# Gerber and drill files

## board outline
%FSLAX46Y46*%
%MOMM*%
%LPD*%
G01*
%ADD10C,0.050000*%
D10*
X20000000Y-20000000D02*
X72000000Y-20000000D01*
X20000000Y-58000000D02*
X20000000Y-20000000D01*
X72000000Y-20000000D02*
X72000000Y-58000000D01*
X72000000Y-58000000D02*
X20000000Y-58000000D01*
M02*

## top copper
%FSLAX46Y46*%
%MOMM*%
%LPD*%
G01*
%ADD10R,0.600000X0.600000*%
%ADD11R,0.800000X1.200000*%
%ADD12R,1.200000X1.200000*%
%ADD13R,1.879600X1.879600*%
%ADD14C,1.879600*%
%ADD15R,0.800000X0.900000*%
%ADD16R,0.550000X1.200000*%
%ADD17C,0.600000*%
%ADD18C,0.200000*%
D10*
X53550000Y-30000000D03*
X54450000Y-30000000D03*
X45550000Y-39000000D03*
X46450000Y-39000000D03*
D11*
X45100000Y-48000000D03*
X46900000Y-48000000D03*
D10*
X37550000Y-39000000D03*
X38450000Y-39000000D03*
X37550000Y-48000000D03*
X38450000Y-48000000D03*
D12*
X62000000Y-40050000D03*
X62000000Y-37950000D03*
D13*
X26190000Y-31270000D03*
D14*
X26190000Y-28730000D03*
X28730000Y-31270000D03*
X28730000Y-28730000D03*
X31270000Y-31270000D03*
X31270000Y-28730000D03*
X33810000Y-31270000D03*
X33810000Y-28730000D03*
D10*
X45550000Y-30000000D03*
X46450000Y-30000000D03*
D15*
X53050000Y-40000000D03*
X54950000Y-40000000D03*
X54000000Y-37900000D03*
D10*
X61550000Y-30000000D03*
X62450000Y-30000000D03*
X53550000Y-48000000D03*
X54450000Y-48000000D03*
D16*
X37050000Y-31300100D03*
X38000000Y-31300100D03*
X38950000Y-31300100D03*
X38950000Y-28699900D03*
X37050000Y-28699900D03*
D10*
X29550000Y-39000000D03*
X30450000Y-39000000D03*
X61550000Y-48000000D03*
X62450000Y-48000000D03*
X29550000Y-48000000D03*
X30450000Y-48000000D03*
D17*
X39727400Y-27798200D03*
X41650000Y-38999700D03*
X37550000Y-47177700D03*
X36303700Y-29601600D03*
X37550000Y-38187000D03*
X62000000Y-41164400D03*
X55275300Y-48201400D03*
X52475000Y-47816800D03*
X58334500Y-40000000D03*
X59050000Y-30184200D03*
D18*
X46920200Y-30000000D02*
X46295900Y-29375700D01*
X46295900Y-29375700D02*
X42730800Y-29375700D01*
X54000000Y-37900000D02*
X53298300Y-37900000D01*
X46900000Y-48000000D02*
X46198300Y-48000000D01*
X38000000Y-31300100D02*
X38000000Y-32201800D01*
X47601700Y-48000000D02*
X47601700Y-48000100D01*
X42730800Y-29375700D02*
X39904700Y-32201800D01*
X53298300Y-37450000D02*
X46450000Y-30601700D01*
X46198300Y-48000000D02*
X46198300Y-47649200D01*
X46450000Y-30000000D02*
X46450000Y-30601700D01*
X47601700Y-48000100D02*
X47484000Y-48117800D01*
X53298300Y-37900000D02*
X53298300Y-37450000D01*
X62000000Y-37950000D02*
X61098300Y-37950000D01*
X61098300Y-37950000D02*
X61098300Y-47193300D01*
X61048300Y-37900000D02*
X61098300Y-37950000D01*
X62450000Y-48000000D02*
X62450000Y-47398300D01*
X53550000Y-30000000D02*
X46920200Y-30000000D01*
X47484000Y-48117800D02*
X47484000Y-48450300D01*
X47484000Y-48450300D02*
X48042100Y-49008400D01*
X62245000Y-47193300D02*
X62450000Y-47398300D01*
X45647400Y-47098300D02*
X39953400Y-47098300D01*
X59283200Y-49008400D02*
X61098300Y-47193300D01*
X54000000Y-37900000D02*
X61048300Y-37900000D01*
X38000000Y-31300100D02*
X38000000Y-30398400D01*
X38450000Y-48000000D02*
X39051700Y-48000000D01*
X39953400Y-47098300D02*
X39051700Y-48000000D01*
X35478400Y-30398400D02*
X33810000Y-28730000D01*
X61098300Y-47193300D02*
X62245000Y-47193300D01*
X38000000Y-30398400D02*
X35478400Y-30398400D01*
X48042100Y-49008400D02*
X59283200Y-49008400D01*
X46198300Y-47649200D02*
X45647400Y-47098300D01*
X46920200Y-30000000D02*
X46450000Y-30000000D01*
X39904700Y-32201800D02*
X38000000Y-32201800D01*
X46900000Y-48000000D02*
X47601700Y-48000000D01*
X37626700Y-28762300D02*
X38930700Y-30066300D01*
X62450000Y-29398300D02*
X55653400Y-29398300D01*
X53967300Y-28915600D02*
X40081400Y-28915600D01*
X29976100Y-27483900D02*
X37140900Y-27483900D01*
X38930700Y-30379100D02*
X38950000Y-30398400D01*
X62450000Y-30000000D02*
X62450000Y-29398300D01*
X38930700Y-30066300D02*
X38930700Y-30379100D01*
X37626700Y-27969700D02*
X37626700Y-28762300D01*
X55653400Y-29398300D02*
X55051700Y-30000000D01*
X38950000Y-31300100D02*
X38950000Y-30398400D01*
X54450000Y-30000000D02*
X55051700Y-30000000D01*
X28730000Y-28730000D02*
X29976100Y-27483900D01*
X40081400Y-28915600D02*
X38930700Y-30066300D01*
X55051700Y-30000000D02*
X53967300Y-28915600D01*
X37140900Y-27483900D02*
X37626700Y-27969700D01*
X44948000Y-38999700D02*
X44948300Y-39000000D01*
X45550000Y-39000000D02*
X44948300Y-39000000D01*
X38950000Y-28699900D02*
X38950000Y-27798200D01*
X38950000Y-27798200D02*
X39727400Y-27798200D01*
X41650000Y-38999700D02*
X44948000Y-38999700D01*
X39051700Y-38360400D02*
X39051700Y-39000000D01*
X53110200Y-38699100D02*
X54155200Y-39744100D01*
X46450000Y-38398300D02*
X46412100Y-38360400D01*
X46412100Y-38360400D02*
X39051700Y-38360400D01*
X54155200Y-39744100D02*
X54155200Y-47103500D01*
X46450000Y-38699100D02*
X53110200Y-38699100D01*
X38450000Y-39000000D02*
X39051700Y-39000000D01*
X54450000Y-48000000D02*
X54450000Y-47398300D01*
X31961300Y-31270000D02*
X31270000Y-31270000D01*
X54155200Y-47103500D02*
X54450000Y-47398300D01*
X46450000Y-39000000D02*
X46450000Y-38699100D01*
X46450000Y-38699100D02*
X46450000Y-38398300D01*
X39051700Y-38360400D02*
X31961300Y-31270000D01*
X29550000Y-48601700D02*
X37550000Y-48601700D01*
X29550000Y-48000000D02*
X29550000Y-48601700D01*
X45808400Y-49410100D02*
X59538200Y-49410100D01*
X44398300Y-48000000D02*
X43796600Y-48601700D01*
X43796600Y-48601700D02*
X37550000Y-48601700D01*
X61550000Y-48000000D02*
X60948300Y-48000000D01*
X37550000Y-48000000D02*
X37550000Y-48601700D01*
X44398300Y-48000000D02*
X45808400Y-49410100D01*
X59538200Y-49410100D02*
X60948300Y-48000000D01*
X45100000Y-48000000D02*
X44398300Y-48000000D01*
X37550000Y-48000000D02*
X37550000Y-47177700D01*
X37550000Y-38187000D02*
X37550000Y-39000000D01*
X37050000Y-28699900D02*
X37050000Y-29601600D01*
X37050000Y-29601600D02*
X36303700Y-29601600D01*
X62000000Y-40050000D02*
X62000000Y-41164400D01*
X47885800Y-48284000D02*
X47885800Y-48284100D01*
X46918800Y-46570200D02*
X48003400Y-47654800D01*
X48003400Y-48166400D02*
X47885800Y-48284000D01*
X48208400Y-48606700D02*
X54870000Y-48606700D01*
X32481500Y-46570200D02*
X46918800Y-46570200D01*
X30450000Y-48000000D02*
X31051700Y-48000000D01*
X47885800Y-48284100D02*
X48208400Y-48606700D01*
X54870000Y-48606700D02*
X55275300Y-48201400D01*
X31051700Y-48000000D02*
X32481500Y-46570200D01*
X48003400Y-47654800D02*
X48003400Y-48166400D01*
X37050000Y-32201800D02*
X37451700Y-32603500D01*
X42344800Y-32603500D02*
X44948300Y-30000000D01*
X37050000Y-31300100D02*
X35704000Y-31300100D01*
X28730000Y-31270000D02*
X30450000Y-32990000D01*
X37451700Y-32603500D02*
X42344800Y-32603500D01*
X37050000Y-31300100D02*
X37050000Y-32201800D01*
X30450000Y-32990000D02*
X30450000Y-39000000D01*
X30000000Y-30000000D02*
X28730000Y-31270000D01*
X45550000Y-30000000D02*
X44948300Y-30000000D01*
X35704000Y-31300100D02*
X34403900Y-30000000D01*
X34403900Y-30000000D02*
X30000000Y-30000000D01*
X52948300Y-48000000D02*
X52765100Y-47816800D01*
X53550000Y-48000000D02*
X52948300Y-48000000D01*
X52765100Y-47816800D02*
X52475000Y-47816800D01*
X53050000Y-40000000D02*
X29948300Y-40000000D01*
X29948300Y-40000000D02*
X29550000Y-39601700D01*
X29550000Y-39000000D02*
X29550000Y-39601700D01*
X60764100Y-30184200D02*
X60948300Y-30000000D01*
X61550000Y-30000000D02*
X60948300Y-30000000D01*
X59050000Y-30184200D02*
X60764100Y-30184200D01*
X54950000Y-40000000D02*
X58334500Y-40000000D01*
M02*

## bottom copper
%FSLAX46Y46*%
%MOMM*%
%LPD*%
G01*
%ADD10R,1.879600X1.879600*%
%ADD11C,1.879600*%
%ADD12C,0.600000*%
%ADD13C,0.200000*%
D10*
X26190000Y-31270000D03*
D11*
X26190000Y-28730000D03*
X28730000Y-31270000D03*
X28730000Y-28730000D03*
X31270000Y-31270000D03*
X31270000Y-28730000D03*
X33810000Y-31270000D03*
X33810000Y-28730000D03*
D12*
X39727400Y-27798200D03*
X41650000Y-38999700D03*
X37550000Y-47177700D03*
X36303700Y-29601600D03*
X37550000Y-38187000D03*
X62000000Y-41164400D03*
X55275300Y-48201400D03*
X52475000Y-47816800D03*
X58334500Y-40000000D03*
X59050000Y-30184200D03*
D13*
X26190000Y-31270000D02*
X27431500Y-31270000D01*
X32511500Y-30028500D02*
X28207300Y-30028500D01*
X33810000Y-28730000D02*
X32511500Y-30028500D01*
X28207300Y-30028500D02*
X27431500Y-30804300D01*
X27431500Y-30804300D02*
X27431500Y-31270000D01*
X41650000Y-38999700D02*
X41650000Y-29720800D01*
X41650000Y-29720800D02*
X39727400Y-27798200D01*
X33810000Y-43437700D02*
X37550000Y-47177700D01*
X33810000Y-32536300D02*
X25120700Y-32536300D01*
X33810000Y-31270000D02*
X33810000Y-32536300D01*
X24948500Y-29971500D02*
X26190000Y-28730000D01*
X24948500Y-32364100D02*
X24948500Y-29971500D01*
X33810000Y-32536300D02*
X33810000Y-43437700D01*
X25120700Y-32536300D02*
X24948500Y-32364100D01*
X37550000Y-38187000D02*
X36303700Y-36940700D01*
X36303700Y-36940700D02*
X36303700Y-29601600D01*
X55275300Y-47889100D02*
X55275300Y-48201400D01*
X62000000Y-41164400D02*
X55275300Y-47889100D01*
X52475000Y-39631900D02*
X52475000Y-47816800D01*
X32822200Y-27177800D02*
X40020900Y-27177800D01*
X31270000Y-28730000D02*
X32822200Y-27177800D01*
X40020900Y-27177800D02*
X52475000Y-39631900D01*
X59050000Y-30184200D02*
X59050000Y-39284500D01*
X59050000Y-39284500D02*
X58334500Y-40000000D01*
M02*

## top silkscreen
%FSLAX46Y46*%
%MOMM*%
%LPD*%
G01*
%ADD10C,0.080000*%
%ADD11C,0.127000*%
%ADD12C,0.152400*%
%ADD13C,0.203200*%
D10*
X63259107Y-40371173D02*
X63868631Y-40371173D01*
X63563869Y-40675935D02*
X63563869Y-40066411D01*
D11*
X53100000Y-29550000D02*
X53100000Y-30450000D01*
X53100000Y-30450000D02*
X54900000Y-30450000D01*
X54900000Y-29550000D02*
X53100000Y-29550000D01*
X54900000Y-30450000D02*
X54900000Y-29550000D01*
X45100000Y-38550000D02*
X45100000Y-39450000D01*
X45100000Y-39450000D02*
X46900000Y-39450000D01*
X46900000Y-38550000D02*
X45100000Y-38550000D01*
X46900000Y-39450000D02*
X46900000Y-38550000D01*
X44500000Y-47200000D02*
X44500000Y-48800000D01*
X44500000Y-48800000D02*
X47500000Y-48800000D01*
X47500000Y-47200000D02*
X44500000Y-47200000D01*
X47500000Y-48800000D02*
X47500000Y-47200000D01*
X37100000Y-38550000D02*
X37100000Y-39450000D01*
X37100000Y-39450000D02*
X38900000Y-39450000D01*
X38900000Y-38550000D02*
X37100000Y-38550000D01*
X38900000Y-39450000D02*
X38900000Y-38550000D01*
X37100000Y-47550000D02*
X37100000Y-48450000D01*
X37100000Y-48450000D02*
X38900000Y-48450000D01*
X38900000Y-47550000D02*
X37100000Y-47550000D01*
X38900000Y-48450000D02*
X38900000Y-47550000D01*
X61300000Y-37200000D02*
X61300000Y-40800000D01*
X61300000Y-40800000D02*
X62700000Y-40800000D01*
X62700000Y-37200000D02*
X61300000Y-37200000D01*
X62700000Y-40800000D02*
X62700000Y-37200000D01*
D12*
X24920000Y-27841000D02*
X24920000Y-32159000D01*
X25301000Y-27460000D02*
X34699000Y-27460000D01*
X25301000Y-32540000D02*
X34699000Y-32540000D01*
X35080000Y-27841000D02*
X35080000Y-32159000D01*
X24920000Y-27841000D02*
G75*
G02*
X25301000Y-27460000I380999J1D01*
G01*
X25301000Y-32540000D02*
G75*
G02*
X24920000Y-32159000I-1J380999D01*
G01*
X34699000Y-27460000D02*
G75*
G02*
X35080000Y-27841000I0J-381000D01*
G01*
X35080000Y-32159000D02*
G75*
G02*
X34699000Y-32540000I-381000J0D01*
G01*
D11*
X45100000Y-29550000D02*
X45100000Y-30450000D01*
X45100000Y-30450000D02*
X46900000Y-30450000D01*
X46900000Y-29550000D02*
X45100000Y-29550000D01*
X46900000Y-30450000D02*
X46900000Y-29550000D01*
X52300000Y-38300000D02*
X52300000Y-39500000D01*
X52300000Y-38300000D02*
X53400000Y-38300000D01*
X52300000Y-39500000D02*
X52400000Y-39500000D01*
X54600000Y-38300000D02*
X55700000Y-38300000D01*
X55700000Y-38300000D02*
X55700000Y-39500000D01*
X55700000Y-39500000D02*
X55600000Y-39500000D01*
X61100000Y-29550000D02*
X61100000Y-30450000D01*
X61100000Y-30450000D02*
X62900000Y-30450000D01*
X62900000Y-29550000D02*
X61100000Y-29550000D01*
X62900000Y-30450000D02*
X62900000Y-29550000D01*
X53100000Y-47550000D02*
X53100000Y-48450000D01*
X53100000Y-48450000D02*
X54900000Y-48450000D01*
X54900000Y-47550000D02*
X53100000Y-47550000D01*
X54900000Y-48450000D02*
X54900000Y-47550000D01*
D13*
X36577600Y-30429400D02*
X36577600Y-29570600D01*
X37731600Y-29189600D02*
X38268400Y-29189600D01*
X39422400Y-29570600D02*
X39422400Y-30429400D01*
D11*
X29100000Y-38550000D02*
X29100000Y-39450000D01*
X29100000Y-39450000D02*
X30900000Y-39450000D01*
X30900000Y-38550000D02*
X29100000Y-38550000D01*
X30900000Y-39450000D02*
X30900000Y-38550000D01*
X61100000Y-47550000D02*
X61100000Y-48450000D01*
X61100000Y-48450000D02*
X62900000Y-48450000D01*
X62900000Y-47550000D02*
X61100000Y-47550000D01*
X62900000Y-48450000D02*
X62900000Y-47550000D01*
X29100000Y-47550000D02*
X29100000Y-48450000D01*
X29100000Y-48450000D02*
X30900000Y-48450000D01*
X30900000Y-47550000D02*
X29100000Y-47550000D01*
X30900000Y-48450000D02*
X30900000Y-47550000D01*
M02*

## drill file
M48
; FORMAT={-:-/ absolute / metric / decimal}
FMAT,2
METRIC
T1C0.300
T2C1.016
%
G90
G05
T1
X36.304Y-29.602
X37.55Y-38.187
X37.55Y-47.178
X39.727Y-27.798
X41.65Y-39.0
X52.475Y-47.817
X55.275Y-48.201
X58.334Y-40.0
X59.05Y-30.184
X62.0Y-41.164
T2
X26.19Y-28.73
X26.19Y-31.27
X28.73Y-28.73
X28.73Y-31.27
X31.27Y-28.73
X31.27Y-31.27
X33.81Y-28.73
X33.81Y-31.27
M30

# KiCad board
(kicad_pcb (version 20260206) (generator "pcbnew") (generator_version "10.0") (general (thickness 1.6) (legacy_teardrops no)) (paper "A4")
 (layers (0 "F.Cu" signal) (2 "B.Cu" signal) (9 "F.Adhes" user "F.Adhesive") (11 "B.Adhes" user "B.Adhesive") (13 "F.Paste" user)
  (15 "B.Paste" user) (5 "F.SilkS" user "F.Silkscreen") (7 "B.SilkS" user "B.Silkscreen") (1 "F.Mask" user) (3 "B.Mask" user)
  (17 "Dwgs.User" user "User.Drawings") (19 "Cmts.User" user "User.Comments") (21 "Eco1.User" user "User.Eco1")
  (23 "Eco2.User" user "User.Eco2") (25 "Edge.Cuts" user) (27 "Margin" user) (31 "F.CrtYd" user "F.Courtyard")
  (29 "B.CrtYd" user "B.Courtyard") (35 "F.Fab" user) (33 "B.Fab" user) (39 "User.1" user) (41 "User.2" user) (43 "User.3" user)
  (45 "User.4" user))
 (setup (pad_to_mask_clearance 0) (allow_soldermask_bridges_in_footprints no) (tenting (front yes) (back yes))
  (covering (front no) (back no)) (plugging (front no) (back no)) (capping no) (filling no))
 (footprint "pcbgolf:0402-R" (layer "F.Cu") (at 54 30)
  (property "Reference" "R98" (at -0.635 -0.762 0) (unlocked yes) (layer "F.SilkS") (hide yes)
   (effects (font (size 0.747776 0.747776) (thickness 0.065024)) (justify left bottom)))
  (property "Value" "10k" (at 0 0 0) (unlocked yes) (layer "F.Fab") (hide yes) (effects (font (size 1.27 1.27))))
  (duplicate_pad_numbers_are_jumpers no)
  (fp_line (start -0.9 -0.45) (end -0.9 0.45) (stroke (width 0.127) (type solid)) (layer "F.SilkS"))
  (fp_line (start -0.9 0.45) (end 0.9 0.45) (stroke (width 0.127) (type solid)) (layer "F.SilkS"))
  (fp_line (start 0.9 -0.45) (end -0.9 -0.45) (stroke (width 0.127) (type solid)) (layer "F.SilkS"))
  (fp_line (start 0.9 0.45) (end 0.9 -0.45) (stroke (width 0.127) (type solid)) (layer "F.SilkS"))
  (pad "1" smd rect (at -0.45 0) (size 0.6 0.6) (layers "F.Cu" "F.Mask" "F.Paste") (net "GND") (solder_mask_margin 0.0508)
   (solder_paste_margin 0) (thermal_bridge_angle 0))
  (pad "2" smd rect (at 0.45 0) (size 0.6 0.6) (layers "F.Cu" "F.Mask" "F.Paste") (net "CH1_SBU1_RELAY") (solder_mask_margin 0.0508)
   (solder_paste_margin 0) (thermal_bridge_angle 0)))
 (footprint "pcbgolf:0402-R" (layer "F.Cu") (at 46 39)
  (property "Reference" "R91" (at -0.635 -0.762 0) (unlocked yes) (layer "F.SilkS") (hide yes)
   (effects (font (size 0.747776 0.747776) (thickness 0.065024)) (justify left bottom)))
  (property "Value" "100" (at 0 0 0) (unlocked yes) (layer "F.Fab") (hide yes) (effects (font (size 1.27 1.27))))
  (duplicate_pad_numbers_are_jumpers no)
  (fp_line (start -0.9 -0.45) (end -0.9 0.45) (stroke (width 0.127) (type solid)) (layer "F.SilkS"))
  (fp_line (start -0.9 0.45) (end 0.9 0.45) (stroke (width 0.127) (type solid)) (layer "F.SilkS"))
  (fp_line (start 0.9 -0.45) (end -0.9 -0.45) (stroke (width 0.127) (type solid)) (layer "F.SilkS"))
  (fp_line (start 0.9 0.45) (end 0.9 -0.45) (stroke (width 0.127) (type solid)) (layer "F.SilkS"))
  (pad "1" smd rect (at -0.45 0) (size 0.6 0.6) (layers "F.Cu" "F.Mask" "F.Paste") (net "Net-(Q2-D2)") (solder_mask_margin 0.0508)
   (solder_paste_margin 0) (thermal_bridge_angle 0))
  (pad "2" smd rect (at 0.45 0) (size 0.6 0.6) (layers "F.Cu" "F.Mask" "F.Paste") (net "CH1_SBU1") (solder_mask_margin 0.0508)
   (solder_paste_margin 0) (thermal_bridge_angle 0)))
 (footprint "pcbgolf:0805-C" (layer "F.Cu") (at 46 48)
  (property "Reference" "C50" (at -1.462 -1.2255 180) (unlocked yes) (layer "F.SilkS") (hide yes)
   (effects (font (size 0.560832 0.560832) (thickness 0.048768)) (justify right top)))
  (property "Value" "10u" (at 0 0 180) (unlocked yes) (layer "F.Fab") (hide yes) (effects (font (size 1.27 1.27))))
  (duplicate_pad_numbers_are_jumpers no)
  (fp_line (start -1.5 -0.8) (end -1.5 0.8) (stroke (width 0.127) (type solid)) (layer "F.SilkS"))
  (fp_line (start -1.5 0.8) (end 1.5 0.8) (stroke (width 0.127) (type solid)) (layer "F.SilkS"))
  (fp_line (start 1.5 -0.8) (end -1.5 -0.8) (stroke (width 0.127) (type solid)) (layer "F.SilkS"))
  (fp_line (start 1.5 0.8) (end 1.5 -0.8) (stroke (width 0.127) (type solid)) (layer "F.SilkS"))
  (pad "1" smd rect (at -0.9 0) (size 0.8 1.2) (layers "F.Cu" "F.Mask" "F.Paste") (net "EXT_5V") (solder_mask_margin 0.0508)
   (solder_paste_margin 0) (thermal_bridge_angle 0))
  (pad "2" smd rect (at 0.9 0) (size 0.8 1.2) (layers "F.Cu" "F.Mask" "F.Paste") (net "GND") (solder_mask_margin 0.0508)
   (solder_paste_margin 0) (thermal_bridge_angle 0)))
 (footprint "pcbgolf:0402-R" (layer "F.Cu") (at 38 39)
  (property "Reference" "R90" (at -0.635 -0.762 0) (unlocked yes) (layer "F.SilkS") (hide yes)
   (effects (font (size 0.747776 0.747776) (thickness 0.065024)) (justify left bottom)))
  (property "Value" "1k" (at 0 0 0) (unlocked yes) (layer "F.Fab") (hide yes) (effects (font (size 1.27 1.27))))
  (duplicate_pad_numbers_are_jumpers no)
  (fp_line (start -0.9 -0.45) (end -0.9 0.45) (stroke (width 0.127) (type solid)) (layer "F.SilkS"))
  (fp_line (start -0.9 0.45) (end 0.9 0.45) (stroke (width 0.127) (type solid)) (layer "F.SilkS"))
  (fp_line (start 0.9 -0.45) (end -0.9 -0.45) (stroke (width 0.127) (type solid)) (layer "F.SilkS"))
  (fp_line (start 0.9 0.45) (end 0.9 -0.45) (stroke (width 0.127) (type solid)) (layer "F.SilkS"))
  (pad "1" smd rect (at -0.45 0) (size 0.6 0.6) (layers "F.Cu" "F.Mask" "F.Paste") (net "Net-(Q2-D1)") (solder_mask_margin 0.0508)
   (solder_paste_margin 0) (thermal_bridge_angle 0))
  (pad "2" smd rect (at 0.45 0) (size 0.6 0.6) (layers "F.Cu" "F.Mask" "F.Paste") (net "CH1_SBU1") (solder_mask_margin 0.0508)
   (solder_paste_margin 0) (thermal_bridge_angle 0)))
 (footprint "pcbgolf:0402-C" (layer "F.Cu") (at 38 48)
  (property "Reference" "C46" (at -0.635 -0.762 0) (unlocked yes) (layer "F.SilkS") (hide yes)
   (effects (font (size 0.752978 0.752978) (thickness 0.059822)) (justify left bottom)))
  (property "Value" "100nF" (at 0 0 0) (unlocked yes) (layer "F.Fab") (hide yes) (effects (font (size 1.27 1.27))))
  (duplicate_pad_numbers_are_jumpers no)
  (fp_line (start -0.9 -0.45) (end -0.9 0.45) (stroke (width 0.127) (type solid)) (layer "F.SilkS"))
  (fp_line (start -0.9 0.45) (end 0.9 0.45) (stroke (width 0.127) (type solid)) (layer "F.SilkS"))
  (fp_line (start 0.9 -0.45) (end -0.9 -0.45) (stroke (width 0.127) (type solid)) (layer "F.SilkS"))
  (fp_line (start 0.9 0.45) (end 0.9 -0.45) (stroke (width 0.127) (type solid)) (layer "F.SilkS"))
  (pad "1" smd rect (at -0.45 0) (size 0.6 0.6) (layers "F.Cu" "F.Mask" "F.Paste") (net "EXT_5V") (solder_mask_margin 0.0508)
   (solder_paste_margin 0) (thermal_bridge_angle 0))
  (pad "2" smd rect (at 0.45 0) (size 0.6 0.6) (layers "F.Cu" "F.Mask" "F.Paste") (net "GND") (solder_mask_margin 0.0508)
   (solder_paste_margin 0) (thermal_bridge_angle 0)))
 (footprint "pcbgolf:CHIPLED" (layer "F.Cu") (at 62 39)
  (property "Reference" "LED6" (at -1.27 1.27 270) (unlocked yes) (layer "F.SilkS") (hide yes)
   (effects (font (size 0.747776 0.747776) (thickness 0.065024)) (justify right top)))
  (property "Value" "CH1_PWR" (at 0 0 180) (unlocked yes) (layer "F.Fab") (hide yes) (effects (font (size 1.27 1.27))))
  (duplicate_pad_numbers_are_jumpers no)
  (fp_line (start -0.7 -1.8) (end -0.7 1.8) (stroke (width 0.127) (type solid)) (layer "F.SilkS"))
  (fp_line (start -0.7 1.8) (end 0.7 1.8) (stroke (width 0.127) (type solid)) (layer "F.SilkS"))
  (fp_line (start 0.7 -1.8) (end -0.7 -1.8) (stroke (width 0.127) (type solid)) (layer "F.SilkS"))
  (fp_line (start 0.7 1.8) (end 0.7 -1.8) (stroke (width 0.127) (type solid)) (layer "F.SilkS"))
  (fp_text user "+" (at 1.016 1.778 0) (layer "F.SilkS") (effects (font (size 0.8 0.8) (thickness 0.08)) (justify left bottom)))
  (pad "A" smd rect (at 0 1.05) (size 1.2 1.2) (layers "F.Cu" "F.Mask" "F.Paste") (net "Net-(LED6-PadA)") (solder_mask_margin 0.0508)
   (solder_paste_margin 0) (thermal_bridge_angle 0))
  (pad "C" smd rect (at 0 -1.05) (size 1.2 1.2) (layers "F.Cu" "F.Mask" "F.Paste") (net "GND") (solder_mask_margin 0.0508)
   (solder_paste_margin 0) (thermal_bridge_angle 0)))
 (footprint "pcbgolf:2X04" (layer "F.Cu") (at 30 30)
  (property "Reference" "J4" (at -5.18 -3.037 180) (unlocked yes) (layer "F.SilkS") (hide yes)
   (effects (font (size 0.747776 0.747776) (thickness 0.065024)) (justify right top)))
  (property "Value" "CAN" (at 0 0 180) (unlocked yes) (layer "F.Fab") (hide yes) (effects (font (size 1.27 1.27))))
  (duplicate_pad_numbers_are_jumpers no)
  (fp_line (start -5.08 -2.159) (end -5.08 2.159) (stroke (width 0.1524) (type solid)) (layer "F.SilkS"))
  (fp_line (start -4.699 -2.54) (end 4.699 -2.54) (stroke (width 0.1524) (type solid)) (layer "F.SilkS"))
  (fp_line (start -4.699 2.54) (end 4.699 2.54) (stroke (width 0.1524) (type solid)) (layer "F.SilkS"))
  (fp_line (start 5.08 -2.159) (end 5.08 2.159) (stroke (width 0.1524) (type solid)) (layer "F.SilkS"))
  (fp_arc (start -5.08 -2.159) (mid -4.968408 -2.428408) (end -4.699 -2.54) (stroke (width 0.1524) (type solid)) (layer "F.SilkS"))
  (fp_arc (start -4.699 2.54) (mid -4.968408 2.428408) (end -5.08 2.159) (stroke (width 0.1524) (type solid)) (layer "F.SilkS"))
  (fp_arc (start 4.699 -2.54) (mid 4.968408 -2.428408) (end 5.08 -2.159) (stroke (width 0.1524) (type solid)) (layer "F.SilkS"))
  (fp_arc (start 5.08 2.159) (mid 4.968408 2.428408) (end 4.699 2.54) (stroke (width 0.1524) (type solid)) (layer "F.SilkS"))
  (pad "1" thru_hole rect (at -3.81 1.27 90) (size 1.8796 1.8796) (drill 1.016) (layers "*.Cu" "*.Mask") (remove_unused_layers no)
   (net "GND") (solder_mask_margin 0.0508) (thermal_bridge_angle 0))
  (pad "2" thru_hole circle (at -3.81 -1.27 90) (size 1.8796 1.8796) (drill 1.016) (layers "*.Cu" "*.Mask") (remove_unused_layers no)
   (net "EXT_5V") (solder_mask_margin 0.0508) (thermal_bridge_angle 0))
  (pad "3" thru_hole circle (at -1.27 1.27 90) (size 1.8796 1.8796) (drill 1.016) (layers "*.Cu" "*.Mask") (remove_unused_layers no)
   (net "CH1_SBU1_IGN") (solder_mask_margin 0.0508) (thermal_bridge_angle 0))
  (pad "4" thru_hole circle (at -1.27 -1.27 90) (size 1.8796 1.8796) (drill 1.016) (layers "*.Cu" "*.Mask") (remove_unused_layers no)
   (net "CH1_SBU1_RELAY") (solder_mask_margin 0.0508) (thermal_bridge_angle 0))
  (pad "5" thru_hole circle (at 1.27 1.27 90) (size 1.8796 1.8796) (drill 1.016) (layers "*.Cu" "*.Mask") (remove_unused_layers no)
   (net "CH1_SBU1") (solder_mask_margin 0.0508) (thermal_bridge_angle 0))
  (pad "6" thru_hole circle (at 1.27 -1.27 90) (size 1.8796 1.8796) (drill 1.016) (layers "*.Cu" "*.Mask") (remove_unused_layers no)
   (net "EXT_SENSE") (solder_mask_margin 0.0508) (thermal_bridge_angle 0))
  (pad "7" thru_hole circle (at 3.81 1.27 90) (size 1.8796 1.8796) (drill 1.016) (layers "*.Cu" "*.Mask") (remove_unused_layers no)
   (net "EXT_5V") (solder_mask_margin 0.0508) (thermal_bridge_angle 0))
  (pad "8" thru_hole circle (at 3.81 -1.27 90) (size 1.8796 1.8796) (drill 1.016) (layers "*.Cu" "*.Mask") (remove_unused_layers no)
   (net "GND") (solder_mask_margin 0.0508) (thermal_bridge_angle 0)))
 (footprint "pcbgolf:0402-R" (layer "F.Cu") (at 46 30)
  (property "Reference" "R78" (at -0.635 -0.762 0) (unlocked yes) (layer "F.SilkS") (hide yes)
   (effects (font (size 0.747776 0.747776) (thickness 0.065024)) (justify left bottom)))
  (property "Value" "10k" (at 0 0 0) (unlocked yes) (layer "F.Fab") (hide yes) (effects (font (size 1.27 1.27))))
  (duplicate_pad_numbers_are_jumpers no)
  (fp_line (start -0.9 -0.45) (end -0.9 0.45) (stroke (width 0.127) (type solid)) (layer "F.SilkS"))
  (fp_line (start -0.9 0.45) (end 0.9 0.45) (stroke (width 0.127) (type solid)) (layer "F.SilkS"))
  (fp_line (start 0.9 -0.45) (end -0.9 -0.45) (stroke (width 0.127) (type solid)) (layer "F.SilkS"))
  (fp_line (start 0.9 0.45) (end 0.9 -0.45) (stroke (width 0.127) (type solid)) (layer "F.SilkS"))
  (pad "1" smd rect (at -0.45 0) (size 0.6 0.6) (layers "F.Cu" "F.Mask" "F.Paste") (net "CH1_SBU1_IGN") (solder_mask_margin 0.0508)
   (solder_paste_margin 0) (thermal_bridge_angle 0))
  (pad "2" smd rect (at 0.45 0) (size 0.6 0.6) (layers "F.Cu" "F.Mask" "F.Paste") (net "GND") (solder_mask_margin 0.0508)
   (solder_paste_margin 0) (thermal_bridge_angle 0)))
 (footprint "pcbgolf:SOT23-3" (layer "F.Cu") (at 54 39)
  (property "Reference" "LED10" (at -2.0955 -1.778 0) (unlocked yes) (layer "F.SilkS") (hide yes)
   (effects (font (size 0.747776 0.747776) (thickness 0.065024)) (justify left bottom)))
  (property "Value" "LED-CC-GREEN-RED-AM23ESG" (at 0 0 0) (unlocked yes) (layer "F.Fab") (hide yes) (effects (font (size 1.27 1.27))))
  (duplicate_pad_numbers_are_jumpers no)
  (fp_line (start -1.7 -0.7) (end -1.7 0.5) (stroke (width 0.127) (type solid)) (layer "F.SilkS"))
  (fp_line (start -1.7 -0.7) (end -0.6 -0.7) (stroke (width 0.127) (type solid)) (layer "F.SilkS"))
  (fp_line (start -1.7 0.5) (end -1.6 0.5) (stroke (width 0.127) (type solid)) (layer "F.SilkS"))
  (fp_line (start 0.6 -0.7) (end 1.7 -0.7) (stroke (width 0.127) (type solid)) (layer "F.SilkS"))
  (fp_line (start 1.7 -0.7) (end 1.7 0.5) (stroke (width 0.127) (type solid)) (layer "F.SilkS"))
  (fp_line (start 1.7 0.5) (end 1.6 0.5) (stroke (width 0.127) (type solid)) (layer "F.SilkS"))
  (pad "1" smd rect (at -0.95 1) (size 0.8 0.9) (layers "F.Cu" "F.Mask" "F.Paste") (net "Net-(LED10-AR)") (solder_mask_margin 0.0508)
   (solder_paste_margin 0) (thermal_bridge_angle 0))
  (pad "2" smd rect (at 0.95 1) (size 0.8 0.9) (layers "F.Cu" "F.Mask" "F.Paste") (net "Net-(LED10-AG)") (solder_mask_margin 0.0508)
   (solder_paste_margin 0) (thermal_bridge_angle 0))
  (pad "3" smd rect (at 0 -1.1) (size 0.8 0.9) (layers "F.Cu" "F.Mask" "F.Paste") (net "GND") (solder_mask_margin 0.0508)
   (solder_paste_margin 0) (thermal_bridge_angle 0)))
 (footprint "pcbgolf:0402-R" (layer "F.Cu") (at 62 30)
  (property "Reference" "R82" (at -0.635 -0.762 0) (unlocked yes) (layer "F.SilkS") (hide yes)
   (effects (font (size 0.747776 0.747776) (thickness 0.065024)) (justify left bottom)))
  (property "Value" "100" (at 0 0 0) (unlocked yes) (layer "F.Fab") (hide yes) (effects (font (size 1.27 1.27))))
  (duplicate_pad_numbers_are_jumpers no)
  (fp_line (start -0.9 -0.45) (end -0.9 0.45) (stroke (width 0.127) (type solid)) (layer "F.SilkS"))
  (fp_line (start -0.9 0.45) (end 0.9 0.45) (stroke (width 0.127) (type solid)) (layer "F.SilkS"))
  (fp_line (start 0.9 -0.45) (end -0.9 -0.45) (stroke (width 0.127) (type solid)) (layer "F.SilkS"))
  (fp_line (start 0.9 0.45) (end 0.9 -0.45) (stroke (width 0.127) (type solid)) (layer "F.SilkS"))
  (pad "1" smd rect (at -0.45 0) (size 0.6 0.6) (layers "F.Cu" "F.Mask" "F.Paste") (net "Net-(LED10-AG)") (solder_mask_margin 0.0508)
   (solder_paste_margin 0) (thermal_bridge_angle 0))
  (pad "2" smd rect (at 0.45 0) (size 0.6 0.6) (layers "F.Cu" "F.Mask" "F.Paste") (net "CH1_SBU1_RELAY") (solder_mask_margin 0.0508)
   (solder_paste_margin 0) (thermal_bridge_angle 0)))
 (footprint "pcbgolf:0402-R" (layer "F.Cu") (at 54 48)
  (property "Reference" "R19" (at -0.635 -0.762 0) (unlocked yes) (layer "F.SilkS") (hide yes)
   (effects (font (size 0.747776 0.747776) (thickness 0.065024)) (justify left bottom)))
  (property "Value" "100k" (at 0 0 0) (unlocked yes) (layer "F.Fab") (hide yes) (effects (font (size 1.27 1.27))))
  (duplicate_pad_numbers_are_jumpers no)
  (fp_line (start -0.9 -0.45) (end -0.9 0.45) (stroke (width 0.127) (type solid)) (layer "F.SilkS"))
  (fp_line (start -0.9 0.45) (end 0.9 0.45) (stroke (width 0.127) (type solid)) (layer "F.SilkS"))
  (fp_line (start 0.9 -0.45) (end -0.9 -0.45) (stroke (width 0.127) (type solid)) (layer "F.SilkS"))
  (fp_line (start 0.9 0.45) (end 0.9 -0.45) (stroke (width 0.127) (type solid)) (layer "F.SilkS"))
  (pad "1" smd rect (at -0.45 0) (size 0.6 0.6) (layers "F.Cu" "F.Mask" "F.Paste") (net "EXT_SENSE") (solder_mask_margin 0.0508)
   (solder_paste_margin 0) (thermal_bridge_angle 0))
  (pad "2" smd rect (at 0.45 0) (size 0.6 0.6) (layers "F.Cu" "F.Mask" "F.Paste") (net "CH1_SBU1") (solder_mask_margin 0.0508)
   (solder_paste_margin 0) (thermal_bridge_angle 0)))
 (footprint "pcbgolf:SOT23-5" (layer "F.Cu") (at 38 30)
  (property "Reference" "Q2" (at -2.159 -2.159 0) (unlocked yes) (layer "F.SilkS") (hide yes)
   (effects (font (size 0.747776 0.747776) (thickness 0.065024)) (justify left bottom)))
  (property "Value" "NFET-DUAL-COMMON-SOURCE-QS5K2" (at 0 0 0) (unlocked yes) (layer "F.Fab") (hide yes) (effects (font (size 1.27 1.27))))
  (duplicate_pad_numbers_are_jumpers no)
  (fp_line (start -1.4224 0.4294) (end -1.4224 -0.4294) (stroke (width 0.2032) (type solid)) (layer "F.SilkS"))
  (fp_line (start -0.2684 -0.8104) (end 0.2684 -0.8104) (stroke (width 0.2032) (type solid)) (layer "F.SilkS"))
  (fp_line (start 1.4224 -0.4294) (end 1.4224 0.4294) (stroke (width 0.2032) (type solid)) (layer "F.SilkS"))
  (pad "1" smd rect (at -0.95 1.3001) (size 0.55 1.2) (layers "F.Cu" "F.Mask" "F.Paste") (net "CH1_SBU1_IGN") (solder_mask_margin 0.0508)
   (solder_paste_margin 0) (thermal_bridge_angle 0))
  (pad "2" smd rect (at 0 1.3001) (size 0.55 1.2) (layers "F.Cu" "F.Mask" "F.Paste") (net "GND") (solder_mask_margin 0.0508)
   (solder_paste_margin 0) (thermal_bridge_angle 0))
  (pad "3" smd rect (at 0.95 1.3001) (size 0.55 1.2) (layers "F.Cu" "F.Mask" "F.Paste") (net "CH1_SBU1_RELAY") (solder_mask_margin 0.0508)
   (solder_paste_margin 0) (thermal_bridge_angle 0))
  (pad "4" smd rect (at 0.95 -1.3001) (size 0.55 1.2) (layers "F.Cu" "F.Mask" "F.Paste") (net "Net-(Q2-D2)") (solder_mask_margin 0.0508)
   (solder_paste_margin 0) (thermal_bridge_angle 0))
  (pad "5" smd rect (at -0.95 -1.3001) (size 0.55 1.2) (layers "F.Cu" "F.Mask" "F.Paste") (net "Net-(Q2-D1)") (solder_mask_margin 0.0508)
   (solder_paste_margin 0) (thermal_bridge_angle 0)))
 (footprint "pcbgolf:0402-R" (layer "F.Cu") (at 30 39)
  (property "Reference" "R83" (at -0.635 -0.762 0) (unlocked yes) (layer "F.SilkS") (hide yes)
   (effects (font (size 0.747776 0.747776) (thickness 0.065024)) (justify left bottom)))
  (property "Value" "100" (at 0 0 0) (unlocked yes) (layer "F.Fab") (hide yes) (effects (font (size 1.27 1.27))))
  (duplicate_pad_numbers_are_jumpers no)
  (fp_line (start -0.9 -0.45) (end -0.9 0.45) (stroke (width 0.127) (type solid)) (layer "F.SilkS"))
  (fp_line (start -0.9 0.45) (end 0.9 0.45) (stroke (width 0.127) (type solid)) (layer "F.SilkS"))
  (fp_line (start 0.9 -0.45) (end -0.9 -0.45) (stroke (width 0.127) (type solid)) (layer "F.SilkS"))
  (fp_line (start 0.9 0.45) (end 0.9 -0.45) (stroke (width 0.127) (type solid)) (layer "F.SilkS"))
  (pad "1" smd rect (at -0.45 0) (size 0.6 0.6) (layers "F.Cu" "F.Mask" "F.Paste") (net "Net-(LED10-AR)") (solder_mask_margin 0.0508)
   (solder_paste_margin 0) (thermal_bridge_angle 0))
  (pad "2" smd rect (at 0.45 0) (size 0.6 0.6) (layers "F.Cu" "F.Mask" "F.Paste") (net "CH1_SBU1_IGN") (solder_mask_margin 0.0508)
   (solder_paste_margin 0) (thermal_bridge_angle 0)))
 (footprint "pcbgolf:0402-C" (layer "F.Cu") (at 62 48)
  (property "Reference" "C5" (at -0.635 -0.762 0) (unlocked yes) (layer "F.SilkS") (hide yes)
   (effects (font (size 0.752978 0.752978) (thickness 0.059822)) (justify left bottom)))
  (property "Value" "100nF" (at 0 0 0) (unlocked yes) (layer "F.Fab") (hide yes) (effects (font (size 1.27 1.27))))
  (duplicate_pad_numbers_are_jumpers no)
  (fp_line (start -0.9 -0.45) (end -0.9 0.45) (stroke (width 0.127) (type solid)) (layer "F.SilkS"))
  (fp_line (start -0.9 0.45) (end 0.9 0.45) (stroke (width 0.127) (type solid)) (layer "F.SilkS"))
  (fp_line (start 0.9 -0.45) (end -0.9 -0.45) (stroke (width 0.127) (type solid)) (layer "F.SilkS"))
  (fp_line (start 0.9 0.45) (end 0.9 -0.45) (stroke (width 0.127) (type solid)) (layer "F.SilkS"))
  (pad "1" smd rect (at -0.45 0) (size 0.6 0.6) (layers "F.Cu" "F.Mask" "F.Paste") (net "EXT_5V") (solder_mask_margin 0.0508)
   (solder_paste_margin 0) (thermal_bridge_angle 0))
  (pad "2" smd rect (at 0.45 0) (size 0.6 0.6) (layers "F.Cu" "F.Mask" "F.Paste") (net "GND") (solder_mask_margin 0.0508)
   (solder_paste_margin 0) (thermal_bridge_angle 0)))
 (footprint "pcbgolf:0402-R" (layer "F.Cu") (at 30 48)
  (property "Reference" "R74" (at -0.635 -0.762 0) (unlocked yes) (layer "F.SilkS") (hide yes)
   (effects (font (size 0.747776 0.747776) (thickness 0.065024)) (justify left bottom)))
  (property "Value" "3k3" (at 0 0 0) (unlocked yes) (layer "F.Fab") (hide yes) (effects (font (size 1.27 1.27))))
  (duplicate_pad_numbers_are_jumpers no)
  (fp_line (start -0.9 -0.45) (end -0.9 0.45) (stroke (width 0.127) (type solid)) (layer "F.SilkS"))
  (fp_line (start -0.9 0.45) (end 0.9 0.45) (stroke (width 0.127) (type solid)) (layer "F.SilkS"))
  (fp_line (start 0.9 -0.45) (end -0.9 -0.45) (stroke (width 0.127) (type solid)) (layer "F.SilkS"))
  (fp_line (start 0.9 0.45) (end 0.9 -0.45) (stroke (width 0.127) (type solid)) (layer "F.SilkS"))
  (pad "1" smd rect (at -0.45 0) (size 0.6 0.6) (layers "F.Cu" "F.Mask" "F.Paste") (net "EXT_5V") (solder_mask_margin 0.0508)
   (solder_paste_margin 0) (thermal_bridge_angle 0))
  (pad "2" smd rect (at 0.45 0) (size 0.6 0.6) (layers "F.Cu" "F.Mask" "F.Paste") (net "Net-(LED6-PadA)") (solder_mask_margin 0.0508)
   (solder_paste_margin 0) (thermal_bridge_angle 0)))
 (gr_line (start 20 20) (end 72 20) (stroke (width 0.05) (type default)) (layer "Edge.Cuts"))
 (gr_line (start 20 58) (end 20 20) (stroke (width 0.05) (type default)) (layer "Edge.Cuts"))
 (gr_line (start 72 20) (end 72 58) (stroke (width 0.05) (type default)) (layer "Edge.Cuts"))
 (gr_line (start 72 58) (end 20 58) (stroke (width 0.05) (type default)) (layer "Edge.Cuts"))
 (segment (start 46.9202 30) (end 46.2959 29.3757) (width 0.2) (layer "F.Cu") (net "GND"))
 (segment (start 46.2959 29.3757) (end 42.7308 29.3757) (width 0.2) (layer "F.Cu") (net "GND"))
 (segment (start 54 37.9) (end 53.2983 37.9) (width 0.2) (layer "F.Cu") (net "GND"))
 (segment (start 46.9 48) (end 46.1983 48) (width 0.2) (layer "F.Cu") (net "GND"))
 (segment (start 38 31.3001) (end 38 32.2018) (width 0.2) (layer "F.Cu") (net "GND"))
 (segment (start 47.6017 48) (end 47.6017 48.0001) (width 0.2) (layer "F.Cu") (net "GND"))
 (segment (start 42.7308 29.3757) (end 39.9047 32.2018) (width 0.2) (layer "F.Cu") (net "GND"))
 (segment (start 53.2983 37.45) (end 46.45 30.6017) (width 0.2) (layer "F.Cu") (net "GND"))
 (segment (start 46.1983 48) (end 46.1983 47.6492) (width 0.2) (layer "F.Cu") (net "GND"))
 (segment (start 46.45 30) (end 46.45 30.6017) (width 0.2) (layer "F.Cu") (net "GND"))
 (segment (start 47.6017 48.0001) (end 47.484 48.1178) (width 0.2) (layer "F.Cu") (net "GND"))
 (segment (start 53.2983 37.9) (end 53.2983 37.45) (width 0.2) (layer "F.Cu") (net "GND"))
 (segment (start 62 37.95) (end 61.0983 37.95) (width 0.2) (layer "F.Cu") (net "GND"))
 (segment (start 61.0983 37.95) (end 61.0983 47.1933) (width 0.2) (layer "F.Cu") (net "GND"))
 (segment (start 61.0483 37.9) (end 61.0983 37.95) (width 0.2) (layer "F.Cu") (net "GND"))
 (segment (start 62.45 48) (end 62.45 47.3983) (width 0.2) (layer "F.Cu") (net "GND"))
 (segment (start 53.55 30) (end 46.9202 30) (width 0.2) (layer "F.Cu") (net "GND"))
 (segment (start 47.484 48.1178) (end 47.484 48.4503) (width 0.2) (layer "F.Cu") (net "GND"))
 (segment (start 47.484 48.4503) (end 48.0421 49.0084) (width 0.2) (layer "F.Cu") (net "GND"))
 (segment (start 62.245 47.1933) (end 62.45 47.3983) (width 0.2) (layer "F.Cu") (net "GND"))
 (segment (start 45.6474 47.0983) (end 39.9534 47.0983) (width 0.2) (layer "F.Cu") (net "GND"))
 (segment (start 59.2832 49.0084) (end 61.0983 47.1933) (width 0.2) (layer "F.Cu") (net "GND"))
 (segment (start 54 37.9) (end 61.0483 37.9) (width 0.2) (layer "F.Cu") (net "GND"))
 (segment (start 38 31.3001) (end 38 30.3984) (width 0.2) (layer "F.Cu") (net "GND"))
 (segment (start 38.45 48) (end 39.0517 48) (width 0.2) (layer "F.Cu") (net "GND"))
 (segment (start 39.9534 47.0983) (end 39.0517 48) (width 0.2) (layer "F.Cu") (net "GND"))
 (segment (start 35.4784 30.3984) (end 33.81 28.73) (width 0.2) (layer "F.Cu") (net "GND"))
 (segment (start 61.0983 47.1933) (end 62.245 47.1933) (width 0.2) (layer "F.Cu") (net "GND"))
 (segment (start 38 30.3984) (end 35.4784 30.3984) (width 0.2) (layer "F.Cu") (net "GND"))
 (segment (start 48.0421 49.0084) (end 59.2832 49.0084) (width 0.2) (layer "F.Cu") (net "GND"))
 (segment (start 46.1983 47.6492) (end 45.6474 47.0983) (width 0.2) (layer "F.Cu") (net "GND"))
 (segment (start 46.9202 30) (end 46.45 30) (width 0.2) (layer "F.Cu") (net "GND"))
 (segment (start 39.9047 32.2018) (end 38 32.2018) (width 0.2) (layer "F.Cu") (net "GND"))
 (segment (start 46.9 48) (end 47.6017 48) (width 0.2) (layer "F.Cu") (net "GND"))
 (segment (start 26.19 31.27) (end 27.4315 31.27) (width 0.2) (layer "B.Cu") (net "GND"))
 (segment (start 32.5115 30.0285) (end 28.2073 30.0285) (width 0.2) (layer "B.Cu") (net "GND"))
 (segment (start 33.81 28.73) (end 32.5115 30.0285) (width 0.2) (layer "B.Cu") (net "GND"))
 (segment (start 28.2073 30.0285) (end 27.4315 30.8043) (width 0.2) (layer "B.Cu") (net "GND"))
 (segment (start 27.4315 30.8043) (end 27.4315 31.27) (width 0.2) (layer "B.Cu") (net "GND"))
 (segment (start 37.6267 28.7623) (end 38.9307 30.0663) (width 0.2) (layer "F.Cu") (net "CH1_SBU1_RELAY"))
 (segment (start 62.45 29.3983) (end 55.6534 29.3983) (width 0.2) (layer "F.Cu") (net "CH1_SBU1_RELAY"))
 (segment (start 53.9673 28.9156) (end 40.0814 28.9156) (width 0.2) (layer "F.Cu") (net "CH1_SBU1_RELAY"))
 (segment (start 29.9761 27.4839) (end 37.1409 27.4839) (width 0.2) (layer "F.Cu") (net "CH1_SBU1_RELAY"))
 (segment (start 38.9307 30.3791) (end 38.95 30.3984) (width 0.2) (layer "F.Cu") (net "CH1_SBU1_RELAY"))
 (segment (start 62.45 30) (end 62.45 29.3983) (width 0.2) (layer "F.Cu") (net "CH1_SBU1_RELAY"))
 (segment (start 38.9307 30.0663) (end 38.9307 30.3791) (width 0.2) (layer "F.Cu") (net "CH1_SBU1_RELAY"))
 (segment (start 37.6267 27.9697) (end 37.6267 28.7623) (width 0.2) (layer "F.Cu") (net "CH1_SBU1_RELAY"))
 (segment (start 55.6534 29.3983) (end 55.0517 30) (width 0.2) (layer "F.Cu") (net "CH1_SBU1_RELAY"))
 (segment (start 38.95 31.3001) (end 38.95 30.3984) (width 0.2) (layer "F.Cu") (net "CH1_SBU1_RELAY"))
 (segment (start 54.45 30) (end 55.0517 30) (width 0.2) (layer "F.Cu") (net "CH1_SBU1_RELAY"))
 (segment (start 28.73 28.73) (end 29.9761 27.4839) (width 0.2) (layer "F.Cu") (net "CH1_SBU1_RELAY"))
 (segment (start 40.0814 28.9156) (end 38.9307 30.0663) (width 0.2) (layer "F.Cu") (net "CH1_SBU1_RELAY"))
 (segment (start 55.0517 30) (end 53.9673 28.9156) (width 0.2) (layer "F.Cu") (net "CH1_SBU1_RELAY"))
 (segment (start 37.1409 27.4839) (end 37.6267 27.9697) (width 0.2) (layer "F.Cu") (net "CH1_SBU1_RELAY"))
 (segment (start 44.948 38.9997) (end 44.9483 39) (width 0.2) (layer "F.Cu") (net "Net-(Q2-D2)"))
 (segment (start 45.55 39) (end 44.9483 39) (width 0.2) (layer "F.Cu") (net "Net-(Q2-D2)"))
 (segment (start 38.95 28.6999) (end 38.95 27.7982) (width 0.2) (layer "F.Cu") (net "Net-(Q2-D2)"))
 (segment (start 38.95 27.7982) (end 39.7274 27.7982) (width 0.2) (layer "F.Cu") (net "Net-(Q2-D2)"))
 (segment (start 41.65 38.9997) (end 44.948 38.9997) (width 0.2) (layer "F.Cu") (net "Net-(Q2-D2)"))
 (via (at 39.7274 27.7982) (size 0.6) (drill 0.3) (layers "F.Cu" "B.Cu") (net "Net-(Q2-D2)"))
 (via (at 41.65 38.9997) (size 0.6) (drill 0.3) (layers "F.Cu" "B.Cu") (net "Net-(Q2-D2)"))
 (segment (start 41.65 38.9997) (end 41.65 29.7208) (width 0.2) (layer "B.Cu") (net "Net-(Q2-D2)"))
 (segment (start 41.65 29.7208) (end 39.7274 27.7982) (width 0.2) (layer "B.Cu") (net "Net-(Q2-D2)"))
 (segment (start 39.0517 38.3604) (end 39.0517 39) (width 0.2) (layer "F.Cu") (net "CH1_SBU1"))
 (segment (start 53.1102 38.6991) (end 54.1552 39.7441) (width 0.2) (layer "F.Cu") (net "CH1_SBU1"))
 (segment (start 46.45 38.3983) (end 46.4121 38.3604) (width 0.2) (layer "F.Cu") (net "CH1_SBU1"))
 (segment (start 46.4121 38.3604) (end 39.0517 38.3604) (width 0.2) (layer "F.Cu") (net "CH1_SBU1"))
 (segment (start 54.1552 39.7441) (end 54.1552 47.1035) (width 0.2) (layer "F.Cu") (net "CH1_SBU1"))
 (segment (start 46.45 38.6991) (end 53.1102 38.6991) (width 0.2) (layer "F.Cu") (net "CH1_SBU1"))
 (segment (start 38.45 39) (end 39.0517 39) (width 0.2) (layer "F.Cu") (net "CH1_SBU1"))
 (segment (start 54.45 48) (end 54.45 47.3983) (width 0.2) (layer "F.Cu") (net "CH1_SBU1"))
 (segment (start 31.9613 31.27) (end 31.27 31.27) (width 0.2) (layer "F.Cu") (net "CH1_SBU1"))
 (segment (start 54.1552 47.1035) (end 54.45 47.3983) (width 0.2) (layer "F.Cu") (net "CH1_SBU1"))
 (segment (start 46.45 39) (end 46.45 38.6991) (width 0.2) (layer "F.Cu") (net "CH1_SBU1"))
 (segment (start 46.45 38.6991) (end 46.45 38.3983) (width 0.2) (layer "F.Cu") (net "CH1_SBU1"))
 (segment (start 39.0517 38.3604) (end 31.9613 31.27) (width 0.2) (layer "F.Cu") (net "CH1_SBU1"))
 (segment (start 29.55 48.6017) (end 37.55 48.6017) (width 0.2) (layer "F.Cu") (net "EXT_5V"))
 (segment (start 29.55 48) (end 29.55 48.6017) (width 0.2) (layer "F.Cu") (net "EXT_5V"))
 (segment (start 45.8084 49.4101) (end 59.5382 49.4101) (width 0.2) (layer "F.Cu") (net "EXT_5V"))
 (segment (start 44.3983 48) (end 43.7966 48.6017) (width 0.2) (layer "F.Cu") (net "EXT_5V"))
 (segment (start 43.7966 48.6017) (end 37.55 48.6017) (width 0.2) (layer "F.Cu") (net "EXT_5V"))
 (segment (start 61.55 48) (end 60.9483 48) (width 0.2) (layer "F.Cu") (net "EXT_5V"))
 (segment (start 37.55 48) (end 37.55 48.6017) (width 0.2) (layer "F.Cu") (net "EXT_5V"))
 (segment (start 44.3983 48) (end 45.8084 49.4101) (width 0.2) (layer "F.Cu") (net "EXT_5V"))
 (segment (start 59.5382 49.4101) (end 60.9483 48) (width 0.2) (layer "F.Cu") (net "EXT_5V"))
 (segment (start 45.1 48) (end 44.3983 48) (width 0.2) (layer "F.Cu") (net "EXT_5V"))
 (segment (start 37.55 48) (end 37.55 47.1777) (width 0.2) (layer "F.Cu") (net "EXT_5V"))
 (via (at 37.55 47.1777) (size 0.6) (drill 0.3) (layers "F.Cu" "B.Cu") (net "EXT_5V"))
 (segment (start 33.81 43.4377) (end 37.55 47.1777) (width 0.2) (layer "B.Cu") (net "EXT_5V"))
 (segment (start 33.81 32.5363) (end 25.1207 32.5363) (width 0.2) (layer "B.Cu") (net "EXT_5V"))
 (segment (start 33.81 31.27) (end 33.81 32.5363) (width 0.2) (layer "B.Cu") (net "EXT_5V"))
 (segment (start 24.9485 29.9715) (end 26.19 28.73) (width 0.2) (layer "B.Cu") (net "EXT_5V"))
 (segment (start 24.9485 32.3641) (end 24.9485 29.9715) (width 0.2) (layer "B.Cu") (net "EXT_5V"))
 (segment (start 33.81 32.5363) (end 33.81 43.4377) (width 0.2) (layer "B.Cu") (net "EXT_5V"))
 (segment (start 25.1207 32.5363) (end 24.9485 32.3641) (width 0.2) (layer "B.Cu") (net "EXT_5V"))
 (segment (start 37.55 38.187) (end 37.55 39) (width 0.2) (layer "F.Cu") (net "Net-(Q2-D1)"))
 (segment (start 37.05 28.6999) (end 37.05 29.6016) (width 0.2) (layer "F.Cu") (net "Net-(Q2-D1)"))
 (segment (start 37.05 29.6016) (end 36.3037 29.6016) (width 0.2) (layer "F.Cu") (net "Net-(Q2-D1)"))
 (via (at 36.3037 29.6016) (size 0.6) (drill 0.3) (layers "F.Cu" "B.Cu") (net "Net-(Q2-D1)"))
 (via (at 37.55 38.187) (size 0.6) (drill 0.3) (layers "F.Cu" "B.Cu") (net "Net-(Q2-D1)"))
 (segment (start 37.55 38.187) (end 36.3037 36.9407) (width 0.2) (layer "B.Cu") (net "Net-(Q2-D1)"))
 (segment (start 36.3037 36.9407) (end 36.3037 29.6016) (width 0.2) (layer "B.Cu") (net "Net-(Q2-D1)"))
 (segment (start 62 40.05) (end 62 41.1644) (width 0.2) (layer "F.Cu") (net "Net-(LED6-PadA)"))
 (segment (start 47.8858 48.284) (end 47.8858 48.2841) (width 0.2) (layer "F.Cu") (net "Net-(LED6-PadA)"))
 (segment (start 46.9188 46.5702) (end 48.0034 47.6548) (width 0.2) (layer "F.Cu") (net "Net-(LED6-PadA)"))
 (segment (start 48.0034 48.1664) (end 47.8858 48.284) (width 0.2) (layer "F.Cu") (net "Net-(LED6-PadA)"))
 (segment (start 48.2084 48.6067) (end 54.87 48.6067) (width 0.2) (layer "F.Cu") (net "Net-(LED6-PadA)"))
 (segment (start 32.4815 46.5702) (end 46.9188 46.5702) (width 0.2) (layer "F.Cu") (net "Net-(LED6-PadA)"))
 (segment (start 30.45 48) (end 31.0517 48) (width 0.2) (layer "F.Cu") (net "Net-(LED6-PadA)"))
 (segment (start 47.8858 48.2841) (end 48.2084 48.6067) (width 0.2) (layer "F.Cu") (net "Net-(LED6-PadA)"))
 (segment (start 54.87 48.6067) (end 55.2753 48.2014) (width 0.2) (layer "F.Cu") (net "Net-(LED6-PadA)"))
 (segment (start 31.0517 48) (end 32.4815 46.5702) (width 0.2) (layer "F.Cu") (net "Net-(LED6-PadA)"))
 (segment (start 48.0034 47.6548) (end 48.0034 48.1664) (width 0.2) (layer "F.Cu") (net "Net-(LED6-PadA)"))
 (via (at 62 41.1644) (size 0.6) (drill 0.3) (layers "F.Cu" "B.Cu") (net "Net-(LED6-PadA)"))
 (via (at 55.2753 48.2014) (size 0.6) (drill 0.3) (layers "F.Cu" "B.Cu") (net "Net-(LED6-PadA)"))
 (segment (start 55.2753 47.8891) (end 55.2753 48.2014) (width 0.2) (layer "B.Cu") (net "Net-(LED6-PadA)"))
 (segment (start 62 41.1644) (end 55.2753 47.8891) (width 0.2) (layer "B.Cu") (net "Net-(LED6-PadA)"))
 (segment (start 37.05 32.2018) (end 37.4517 32.6035) (width 0.2) (layer "F.Cu") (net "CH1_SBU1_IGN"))
 (segment (start 42.3448 32.6035) (end 44.9483 30) (width 0.2) (layer "F.Cu") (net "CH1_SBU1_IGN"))
 (segment (start 37.05 31.3001) (end 35.704 31.3001) (width 0.2) (layer "F.Cu") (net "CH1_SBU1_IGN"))
 (segment (start 28.73 31.27) (end 30.45 32.99) (width 0.2) (layer "F.Cu") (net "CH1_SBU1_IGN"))
 (segment (start 37.4517 32.6035) (end 42.3448 32.6035) (width 0.2) (layer "F.Cu") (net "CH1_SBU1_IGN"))
 (segment (start 37.05 31.3001) (end 37.05 32.2018) (width 0.2) (layer "F.Cu") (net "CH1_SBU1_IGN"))
 (segment (start 30.45 32.99) (end 30.45 39) (width 0.2) (layer "F.Cu") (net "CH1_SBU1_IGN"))
 (segment (start 30 30) (end 28.73 31.27) (width 0.2) (layer "F.Cu") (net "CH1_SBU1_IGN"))
 (segment (start 45.55 30) (end 44.9483 30) (width 0.2) (layer "F.Cu") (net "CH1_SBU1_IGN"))
 (segment (start 35.704 31.3001) (end 34.4039 30) (width 0.2) (layer "F.Cu") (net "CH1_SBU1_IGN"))
 (segment (start 34.4039 30) (end 30 30) (width 0.2) (layer "F.Cu") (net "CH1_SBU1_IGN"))
 (segment (start 52.9483 48) (end 52.7651 47.8168) (width 0.2) (layer "F.Cu") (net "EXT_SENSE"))
 (segment (start 53.55 48) (end 52.9483 48) (width 0.2) (layer "F.Cu") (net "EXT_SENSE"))
 (segment (start 52.7651 47.8168) (end 52.475 47.8168) (width 0.2) (layer "F.Cu") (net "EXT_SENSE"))
 (via (at 52.475 47.8168) (size 0.6) (drill 0.3) (layers "F.Cu" "B.Cu") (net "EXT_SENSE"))
 (segment (start 52.475 39.6319) (end 52.475 47.8168) (width 0.2) (layer "B.Cu") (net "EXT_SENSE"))
 (segment (start 32.8222 27.1778) (end 40.0209 27.1778) (width 0.2) (layer "B.Cu") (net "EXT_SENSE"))
 (segment (start 31.27 28.73) (end 32.8222 27.1778) (width 0.2) (layer "B.Cu") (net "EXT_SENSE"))
 (segment (start 40.0209 27.1778) (end 52.475 39.6319) (width 0.2) (layer "B.Cu") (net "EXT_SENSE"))
 (segment (start 53.05 40) (end 29.9483 40) (width 0.2) (layer "F.Cu") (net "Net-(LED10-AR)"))
 (segment (start 29.9483 40) (end 29.55 39.6017) (width 0.2) (layer "F.Cu") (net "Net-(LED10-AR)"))
 (segment (start 29.55 39) (end 29.55 39.6017) (width 0.2) (layer "F.Cu") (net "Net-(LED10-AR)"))
 (segment (start 60.7641 30.1842) (end 60.9483 30) (width 0.2) (layer "F.Cu") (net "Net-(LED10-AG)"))
 (segment (start 61.55 30) (end 60.9483 30) (width 0.2) (layer "F.Cu") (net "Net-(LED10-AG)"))
 (segment (start 59.05 30.1842) (end 60.7641 30.1842) (width 0.2) (layer "F.Cu") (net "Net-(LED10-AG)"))
 (segment (start 54.95 40) (end 58.3345 40) (width 0.2) (layer "F.Cu") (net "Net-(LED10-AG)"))
 (via (at 58.3345 40) (size 0.6) (drill 0.3) (layers "F.Cu" "B.Cu") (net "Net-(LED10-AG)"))
 (via (at 59.05 30.1842) (size 0.6) (drill 0.3) (layers "F.Cu" "B.Cu") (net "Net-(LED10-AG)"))
 (segment (start 59.05 30.1842) (end 59.05 39.2845) (width 0.2) (layer "B.Cu") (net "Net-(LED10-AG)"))
 (segment (start 59.05 39.2845) (end 58.3345 40) (width 0.2) (layer "B.Cu") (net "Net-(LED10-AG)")))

